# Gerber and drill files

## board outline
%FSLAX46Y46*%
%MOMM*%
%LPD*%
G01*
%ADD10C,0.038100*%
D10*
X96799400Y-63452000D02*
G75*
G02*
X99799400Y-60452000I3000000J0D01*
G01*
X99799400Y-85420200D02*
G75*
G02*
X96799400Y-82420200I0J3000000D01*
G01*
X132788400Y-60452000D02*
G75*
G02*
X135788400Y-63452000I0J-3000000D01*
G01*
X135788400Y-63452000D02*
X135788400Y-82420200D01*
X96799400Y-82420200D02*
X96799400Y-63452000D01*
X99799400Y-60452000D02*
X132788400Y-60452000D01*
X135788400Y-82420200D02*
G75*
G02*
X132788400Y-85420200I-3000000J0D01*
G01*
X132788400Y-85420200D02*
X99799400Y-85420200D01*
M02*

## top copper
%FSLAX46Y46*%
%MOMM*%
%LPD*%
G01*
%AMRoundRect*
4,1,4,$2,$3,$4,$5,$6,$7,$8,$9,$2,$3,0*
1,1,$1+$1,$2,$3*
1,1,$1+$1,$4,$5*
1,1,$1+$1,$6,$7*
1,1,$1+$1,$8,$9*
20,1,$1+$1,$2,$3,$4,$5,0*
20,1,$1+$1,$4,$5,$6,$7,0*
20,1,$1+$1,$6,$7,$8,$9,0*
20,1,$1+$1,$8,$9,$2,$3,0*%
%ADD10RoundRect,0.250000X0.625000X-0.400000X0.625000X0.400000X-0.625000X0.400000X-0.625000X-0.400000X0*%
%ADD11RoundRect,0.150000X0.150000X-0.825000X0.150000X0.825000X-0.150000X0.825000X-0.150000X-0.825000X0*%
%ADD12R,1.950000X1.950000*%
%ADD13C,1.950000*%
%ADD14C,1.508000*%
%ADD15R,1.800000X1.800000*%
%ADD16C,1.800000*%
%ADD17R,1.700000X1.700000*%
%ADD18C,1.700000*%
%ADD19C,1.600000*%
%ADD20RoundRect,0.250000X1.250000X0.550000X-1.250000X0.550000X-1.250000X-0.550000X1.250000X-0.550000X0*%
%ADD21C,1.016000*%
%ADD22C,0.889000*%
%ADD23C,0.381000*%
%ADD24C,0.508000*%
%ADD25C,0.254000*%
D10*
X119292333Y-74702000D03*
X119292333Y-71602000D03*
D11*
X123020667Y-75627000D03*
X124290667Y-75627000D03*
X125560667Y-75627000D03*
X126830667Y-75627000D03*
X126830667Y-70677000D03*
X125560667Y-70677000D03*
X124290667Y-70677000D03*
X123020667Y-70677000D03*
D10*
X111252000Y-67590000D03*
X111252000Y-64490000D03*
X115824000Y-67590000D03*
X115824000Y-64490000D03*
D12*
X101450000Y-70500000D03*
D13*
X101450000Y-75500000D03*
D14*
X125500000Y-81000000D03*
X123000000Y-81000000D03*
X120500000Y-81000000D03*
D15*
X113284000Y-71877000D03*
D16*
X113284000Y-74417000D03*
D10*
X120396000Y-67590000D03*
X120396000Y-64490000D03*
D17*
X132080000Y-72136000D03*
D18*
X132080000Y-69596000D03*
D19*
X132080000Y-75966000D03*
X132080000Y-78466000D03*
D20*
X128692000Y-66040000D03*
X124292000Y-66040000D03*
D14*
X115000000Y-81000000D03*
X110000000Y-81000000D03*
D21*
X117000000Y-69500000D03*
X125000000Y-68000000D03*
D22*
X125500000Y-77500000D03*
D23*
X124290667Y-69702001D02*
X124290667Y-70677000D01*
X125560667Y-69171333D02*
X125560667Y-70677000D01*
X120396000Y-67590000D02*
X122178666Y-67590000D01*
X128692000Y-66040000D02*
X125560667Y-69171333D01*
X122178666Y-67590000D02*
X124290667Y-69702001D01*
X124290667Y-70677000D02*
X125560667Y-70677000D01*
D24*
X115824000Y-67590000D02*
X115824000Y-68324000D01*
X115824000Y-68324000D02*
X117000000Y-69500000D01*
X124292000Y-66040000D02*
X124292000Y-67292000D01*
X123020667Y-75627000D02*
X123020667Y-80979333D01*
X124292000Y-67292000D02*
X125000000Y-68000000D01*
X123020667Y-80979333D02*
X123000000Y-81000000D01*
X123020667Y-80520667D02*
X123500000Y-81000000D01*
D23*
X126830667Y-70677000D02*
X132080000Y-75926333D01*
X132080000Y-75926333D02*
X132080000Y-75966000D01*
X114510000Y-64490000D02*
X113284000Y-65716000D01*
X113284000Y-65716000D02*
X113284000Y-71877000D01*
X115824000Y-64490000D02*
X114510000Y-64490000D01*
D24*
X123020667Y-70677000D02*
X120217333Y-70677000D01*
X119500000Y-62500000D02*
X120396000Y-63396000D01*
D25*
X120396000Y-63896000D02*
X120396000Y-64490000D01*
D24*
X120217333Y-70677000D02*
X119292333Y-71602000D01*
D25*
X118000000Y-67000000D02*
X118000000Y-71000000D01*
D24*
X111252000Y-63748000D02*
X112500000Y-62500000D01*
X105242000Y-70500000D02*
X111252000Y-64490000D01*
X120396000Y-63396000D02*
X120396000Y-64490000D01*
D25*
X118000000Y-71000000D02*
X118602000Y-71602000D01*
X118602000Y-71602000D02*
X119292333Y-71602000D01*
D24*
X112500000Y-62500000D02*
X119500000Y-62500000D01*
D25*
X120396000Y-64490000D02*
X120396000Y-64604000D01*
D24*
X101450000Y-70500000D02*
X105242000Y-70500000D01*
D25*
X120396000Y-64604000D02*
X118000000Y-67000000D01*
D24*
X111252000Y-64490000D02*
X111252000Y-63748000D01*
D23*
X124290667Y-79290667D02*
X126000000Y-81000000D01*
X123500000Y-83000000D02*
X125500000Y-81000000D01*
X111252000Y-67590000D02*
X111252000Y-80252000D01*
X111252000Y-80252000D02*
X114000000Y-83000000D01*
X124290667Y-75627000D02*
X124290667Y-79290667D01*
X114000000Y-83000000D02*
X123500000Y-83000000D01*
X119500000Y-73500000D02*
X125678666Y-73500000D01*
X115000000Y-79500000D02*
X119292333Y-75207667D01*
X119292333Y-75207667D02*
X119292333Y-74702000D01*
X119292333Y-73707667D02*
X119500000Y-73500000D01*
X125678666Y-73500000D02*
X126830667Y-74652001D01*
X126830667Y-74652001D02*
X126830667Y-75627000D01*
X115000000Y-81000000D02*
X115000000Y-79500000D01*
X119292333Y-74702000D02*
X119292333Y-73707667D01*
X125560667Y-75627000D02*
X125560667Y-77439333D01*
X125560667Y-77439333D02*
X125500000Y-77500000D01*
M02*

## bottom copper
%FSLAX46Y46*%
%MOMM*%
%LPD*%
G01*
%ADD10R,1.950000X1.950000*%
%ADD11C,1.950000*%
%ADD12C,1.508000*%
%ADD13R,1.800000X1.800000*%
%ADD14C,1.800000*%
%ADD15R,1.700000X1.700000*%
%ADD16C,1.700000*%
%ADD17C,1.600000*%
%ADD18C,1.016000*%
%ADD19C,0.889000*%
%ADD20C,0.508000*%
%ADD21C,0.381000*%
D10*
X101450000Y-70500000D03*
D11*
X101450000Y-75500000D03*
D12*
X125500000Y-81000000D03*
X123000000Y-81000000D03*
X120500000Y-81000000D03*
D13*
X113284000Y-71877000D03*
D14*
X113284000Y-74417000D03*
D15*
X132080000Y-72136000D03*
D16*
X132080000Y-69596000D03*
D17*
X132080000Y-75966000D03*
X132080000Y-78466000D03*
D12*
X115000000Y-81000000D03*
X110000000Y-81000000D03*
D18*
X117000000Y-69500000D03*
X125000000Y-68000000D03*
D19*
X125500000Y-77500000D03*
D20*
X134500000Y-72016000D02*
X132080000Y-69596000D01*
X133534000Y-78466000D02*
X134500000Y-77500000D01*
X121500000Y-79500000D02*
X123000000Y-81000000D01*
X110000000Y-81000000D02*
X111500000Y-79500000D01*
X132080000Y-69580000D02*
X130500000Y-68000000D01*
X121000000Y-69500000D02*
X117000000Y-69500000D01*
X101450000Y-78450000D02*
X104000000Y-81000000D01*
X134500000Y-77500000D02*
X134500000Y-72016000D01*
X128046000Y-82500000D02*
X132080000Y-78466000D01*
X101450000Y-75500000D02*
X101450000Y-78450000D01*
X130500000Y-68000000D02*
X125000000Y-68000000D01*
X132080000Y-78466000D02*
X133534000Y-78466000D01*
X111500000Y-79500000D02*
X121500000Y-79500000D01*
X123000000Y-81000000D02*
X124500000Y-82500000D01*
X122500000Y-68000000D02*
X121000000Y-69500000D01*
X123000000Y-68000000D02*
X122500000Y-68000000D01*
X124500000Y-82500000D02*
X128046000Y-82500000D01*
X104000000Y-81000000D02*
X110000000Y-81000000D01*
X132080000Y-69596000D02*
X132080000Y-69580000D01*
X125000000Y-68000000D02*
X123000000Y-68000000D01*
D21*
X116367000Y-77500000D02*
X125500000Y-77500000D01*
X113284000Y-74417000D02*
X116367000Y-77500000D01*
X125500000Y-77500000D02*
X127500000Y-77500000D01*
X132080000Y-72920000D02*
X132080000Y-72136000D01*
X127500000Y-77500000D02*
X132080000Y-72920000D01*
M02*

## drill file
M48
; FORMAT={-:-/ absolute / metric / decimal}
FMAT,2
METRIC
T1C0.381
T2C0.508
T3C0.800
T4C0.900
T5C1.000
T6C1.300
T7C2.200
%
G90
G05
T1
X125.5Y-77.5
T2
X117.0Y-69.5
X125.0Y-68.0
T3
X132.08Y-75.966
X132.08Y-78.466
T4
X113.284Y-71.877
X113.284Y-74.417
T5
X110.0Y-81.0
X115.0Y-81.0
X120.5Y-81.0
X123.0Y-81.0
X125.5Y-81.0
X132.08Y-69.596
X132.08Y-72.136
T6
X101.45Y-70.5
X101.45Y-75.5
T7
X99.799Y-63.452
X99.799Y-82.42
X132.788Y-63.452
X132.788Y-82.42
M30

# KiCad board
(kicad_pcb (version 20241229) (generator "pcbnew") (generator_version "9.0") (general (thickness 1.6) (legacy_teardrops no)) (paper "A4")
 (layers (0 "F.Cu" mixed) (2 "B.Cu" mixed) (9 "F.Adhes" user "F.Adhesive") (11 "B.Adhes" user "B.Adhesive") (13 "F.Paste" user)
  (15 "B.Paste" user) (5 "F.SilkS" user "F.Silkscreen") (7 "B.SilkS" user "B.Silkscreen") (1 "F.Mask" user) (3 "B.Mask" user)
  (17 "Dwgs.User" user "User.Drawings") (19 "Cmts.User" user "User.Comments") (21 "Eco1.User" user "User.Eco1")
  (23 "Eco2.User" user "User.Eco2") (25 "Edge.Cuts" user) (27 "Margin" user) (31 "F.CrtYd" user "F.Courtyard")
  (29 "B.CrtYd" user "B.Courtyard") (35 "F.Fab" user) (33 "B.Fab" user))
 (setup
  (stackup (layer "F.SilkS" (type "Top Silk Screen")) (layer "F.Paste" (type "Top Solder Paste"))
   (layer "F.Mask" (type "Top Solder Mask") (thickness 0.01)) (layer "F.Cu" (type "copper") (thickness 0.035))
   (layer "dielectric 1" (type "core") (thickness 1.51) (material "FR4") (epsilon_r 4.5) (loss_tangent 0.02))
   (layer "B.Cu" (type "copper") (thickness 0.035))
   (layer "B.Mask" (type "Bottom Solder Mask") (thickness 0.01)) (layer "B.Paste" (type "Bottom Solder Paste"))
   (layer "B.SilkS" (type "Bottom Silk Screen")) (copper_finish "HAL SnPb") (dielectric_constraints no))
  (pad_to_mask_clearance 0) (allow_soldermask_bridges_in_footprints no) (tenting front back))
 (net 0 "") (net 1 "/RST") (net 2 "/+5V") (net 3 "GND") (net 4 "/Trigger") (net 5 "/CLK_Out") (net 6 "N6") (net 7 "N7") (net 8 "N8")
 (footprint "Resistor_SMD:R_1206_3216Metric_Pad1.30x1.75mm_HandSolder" (layer "F.Cu") (at 119.292333 73.152 90)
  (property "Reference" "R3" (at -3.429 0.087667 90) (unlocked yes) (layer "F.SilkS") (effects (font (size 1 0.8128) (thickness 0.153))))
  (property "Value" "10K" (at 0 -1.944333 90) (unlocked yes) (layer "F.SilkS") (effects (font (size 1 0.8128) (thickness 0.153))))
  (pad "1" smd roundrect (at -1.55 0 90) (size 1.3 1.75) (layers "F.Cu" "F.Mask" "F.Paste") (roundrect_rratio 0.192308) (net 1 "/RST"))
  (pad "2" smd roundrect (at 1.55 0 90) (size 1.3 1.75) (layers "F.Cu" "F.Mask" "F.Paste") (roundrect_rratio 0.192308) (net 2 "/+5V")))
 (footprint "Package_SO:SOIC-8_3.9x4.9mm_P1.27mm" (layer "F.Cu") (at 124.925667 73.152 90)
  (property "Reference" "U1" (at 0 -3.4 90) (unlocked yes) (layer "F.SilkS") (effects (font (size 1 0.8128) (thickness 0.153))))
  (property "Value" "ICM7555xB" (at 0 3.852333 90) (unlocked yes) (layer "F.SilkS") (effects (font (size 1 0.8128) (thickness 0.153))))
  (pad "1" smd roundrect (at -2.475 -1.905 90) (size 1.95 0.6) (layers "F.Cu" "F.Mask" "F.Paste") (roundrect_rratio 0.25) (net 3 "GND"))
  (pad "2" smd roundrect (at -2.475 -0.635 90) (size 1.95 0.6) (layers "F.Cu" "F.Mask" "F.Paste") (roundrect_rratio 0.25) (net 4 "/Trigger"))
  (pad "3" smd roundrect (at -2.475 0.635 90) (size 1.95 0.6) (layers "F.Cu" "F.Mask" "F.Paste") (roundrect_rratio 0.25) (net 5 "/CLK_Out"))
  (pad "4" smd roundrect (at -2.475 1.905 90) (size 1.95 0.6) (layers "F.Cu" "F.Mask" "F.Paste") (roundrect_rratio 0.25) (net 1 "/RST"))
  (pad "5" smd roundrect (at 2.475 1.905 90) (size 1.95 0.6) (layers "F.Cu" "F.Mask" "F.Paste") (roundrect_rratio 0.25) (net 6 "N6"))
  (pad "6" smd roundrect (at 2.475 0.635 90) (size 1.95 0.6) (layers "F.Cu" "F.Mask" "F.Paste") (roundrect_rratio 0.25) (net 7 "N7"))
  (pad "7" smd roundrect (at 2.475 -0.635 90) (size 1.95 0.6) (layers "F.Cu" "F.Mask" "F.Paste") (roundrect_rratio 0.25) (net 7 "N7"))
  (pad "8" smd roundrect (at 2.475 -1.905 90) (size 1.95 0.6) (layers "F.Cu" "F.Mask" "F.Paste") (roundrect_rratio 0.25) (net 2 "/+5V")))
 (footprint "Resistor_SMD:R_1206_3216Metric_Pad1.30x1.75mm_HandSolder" (layer "F.Cu") (at 111.252 66.04 90)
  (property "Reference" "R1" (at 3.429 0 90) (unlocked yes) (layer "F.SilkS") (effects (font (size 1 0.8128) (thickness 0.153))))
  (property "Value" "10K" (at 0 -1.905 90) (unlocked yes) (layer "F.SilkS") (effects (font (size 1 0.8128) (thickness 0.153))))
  (pad "1" smd roundrect (at -1.55 0 90) (size 1.3 1.75) (layers "F.Cu" "F.Mask" "F.Paste") (roundrect_rratio 0.192308) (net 4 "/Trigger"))
  (pad "2" smd roundrect (at 1.55 0 90) (size 1.3 1.75) (layers "F.Cu" "F.Mask" "F.Paste") (roundrect_rratio 0.192308) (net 2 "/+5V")))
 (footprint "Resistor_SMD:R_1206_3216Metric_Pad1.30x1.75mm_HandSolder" (layer "F.Cu") (at 115.824 66.04 90)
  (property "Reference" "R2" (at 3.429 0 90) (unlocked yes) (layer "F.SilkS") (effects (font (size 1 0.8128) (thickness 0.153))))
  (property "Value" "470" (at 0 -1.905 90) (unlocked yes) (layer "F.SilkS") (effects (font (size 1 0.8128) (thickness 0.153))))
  (pad "1" smd roundrect (at -1.55 0 90) (size 1.3 1.75) (layers "F.Cu" "F.Mask" "F.Paste") (roundrect_rratio 0.192308) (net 3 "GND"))
  (pad "2" smd roundrect (at 1.55 0 90) (size 1.3 1.75) (layers "F.Cu" "F.Mask" "F.Paste") (roundrect_rratio 0.192308) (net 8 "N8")))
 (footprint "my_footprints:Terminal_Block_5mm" (layer "F.Cu") (at 101.45 73 -90)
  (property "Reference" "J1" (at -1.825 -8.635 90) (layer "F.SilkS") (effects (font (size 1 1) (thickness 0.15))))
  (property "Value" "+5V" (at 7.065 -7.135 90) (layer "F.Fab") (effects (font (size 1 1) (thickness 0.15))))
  (pad "1" thru_hole rect (at -2.5 0 270) (size 1.95 1.95) (drill 1.3) (layers "*.Cu" "*.Mask") (remove_unused_layers no) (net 2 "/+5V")
   (solder_mask_margin 0.102))
  (pad "2" thru_hole circle (at 2.5 0 270) (size 1.95 1.95) (drill 1.3) (layers "*.Cu" "*.Mask") (remove_unused_layers no) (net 3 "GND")
   (solder_mask_margin 0.102)))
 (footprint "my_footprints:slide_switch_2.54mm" (layer "F.Cu") (at 123 81 180)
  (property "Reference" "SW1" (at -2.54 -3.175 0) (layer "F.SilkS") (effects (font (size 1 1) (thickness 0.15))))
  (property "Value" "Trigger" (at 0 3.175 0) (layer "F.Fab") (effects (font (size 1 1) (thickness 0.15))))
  (pad "1" thru_hole circle (at -2.5 0 180) (size 1.508 1.508) (drill 1) (layers "*.Cu" "*.Mask") (remove_unused_layers no)
   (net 4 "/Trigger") (solder_mask_margin 0.102))
  (pad "2" thru_hole circle (at 0 0 180) (size 1.508 1.508) (drill 1) (layers "*.Cu" "*.Mask") (remove_unused_layers no) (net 3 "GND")
   (solder_mask_margin 0.102))
  (pad "3" thru_hole circle (at 2.5 0 180) (size 1.508 1.508) (drill 1) (layers "*.Cu" "*.Mask") (remove_unused_layers no)
   (solder_mask_margin 0.102)))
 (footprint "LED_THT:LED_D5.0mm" (layer "F.Cu") (at 113.284 71.877 -90)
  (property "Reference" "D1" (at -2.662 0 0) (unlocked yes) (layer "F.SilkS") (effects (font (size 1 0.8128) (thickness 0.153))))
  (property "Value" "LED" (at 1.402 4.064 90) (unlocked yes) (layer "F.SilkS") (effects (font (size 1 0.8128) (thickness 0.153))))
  (pad "1" thru_hole rect (at 0 0 270) (size 1.8 1.8) (drill 0.9) (layers "*.Cu" "*.Mask") (remove_unused_layers no) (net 8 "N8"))
  (pad "2" thru_hole circle (at 2.54 0 270) (size 1.8 1.8) (drill 0.9) (layers "*.Cu" "*.Mask") (remove_unused_layers no) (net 5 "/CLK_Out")))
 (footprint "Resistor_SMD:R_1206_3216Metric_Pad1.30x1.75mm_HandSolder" (layer "F.Cu") (at 120.396 66.04 90)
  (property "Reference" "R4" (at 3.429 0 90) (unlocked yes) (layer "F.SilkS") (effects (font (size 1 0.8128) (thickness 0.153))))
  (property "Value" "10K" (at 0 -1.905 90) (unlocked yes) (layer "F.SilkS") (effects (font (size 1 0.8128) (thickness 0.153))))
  (pad "1" smd roundrect (at -1.55 0 90) (size 1.3 1.75) (layers "F.Cu" "F.Mask" "F.Paste") (roundrect_rratio 0.192308) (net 7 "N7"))
  (pad "2" smd roundrect (at 1.55 0 90) (size 1.3 1.75) (layers "F.Cu" "F.Mask" "F.Paste") (roundrect_rratio 0.192308) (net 2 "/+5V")))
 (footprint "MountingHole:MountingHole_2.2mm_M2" (layer "F.Cu") (at 99.7994 63.452)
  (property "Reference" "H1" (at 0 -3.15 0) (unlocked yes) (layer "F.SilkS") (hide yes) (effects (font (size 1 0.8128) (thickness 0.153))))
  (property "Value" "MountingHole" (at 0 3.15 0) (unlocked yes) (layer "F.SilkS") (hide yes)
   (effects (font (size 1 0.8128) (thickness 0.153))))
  (pad "" np_thru_hole circle (at 0 0) (size 2.2 2.2) (drill 2.2) (layers "*.Cu" "*.Mask")))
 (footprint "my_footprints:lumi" (layer "F.Cu") (at 105.5 63.5)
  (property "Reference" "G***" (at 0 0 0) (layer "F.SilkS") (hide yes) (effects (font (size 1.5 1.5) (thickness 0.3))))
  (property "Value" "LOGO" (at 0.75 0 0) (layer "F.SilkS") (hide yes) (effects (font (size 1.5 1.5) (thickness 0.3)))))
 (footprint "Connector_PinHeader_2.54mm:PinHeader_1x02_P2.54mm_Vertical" (layer "F.Cu") (at 132.08 72.136 180)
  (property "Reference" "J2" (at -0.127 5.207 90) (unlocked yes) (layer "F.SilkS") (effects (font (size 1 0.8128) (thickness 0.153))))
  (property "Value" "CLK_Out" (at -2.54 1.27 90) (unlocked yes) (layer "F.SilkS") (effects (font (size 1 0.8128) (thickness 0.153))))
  (pad "1" thru_hole rect (at 0 0 180) (size 1.7 1.7) (drill 1) (layers "*.Cu" "*.Mask") (remove_unused_layers no) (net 5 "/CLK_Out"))
  (pad "2" thru_hole circle (at 0 2.54 180) (size 1.7 1.7) (drill 1) (layers "*.Cu" "*.Mask") (remove_unused_layers no) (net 3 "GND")))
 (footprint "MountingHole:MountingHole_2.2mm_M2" (layer "F.Cu") (at 132.7884 82.4202)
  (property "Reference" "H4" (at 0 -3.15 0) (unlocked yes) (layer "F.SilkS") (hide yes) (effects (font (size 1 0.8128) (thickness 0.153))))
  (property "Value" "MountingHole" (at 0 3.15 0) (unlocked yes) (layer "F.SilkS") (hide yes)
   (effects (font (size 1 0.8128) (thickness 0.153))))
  (pad "" np_thru_hole circle (at 0 0) (size 2.2 2.2) (drill 2.2) (layers "*.Cu" "*.Mask")))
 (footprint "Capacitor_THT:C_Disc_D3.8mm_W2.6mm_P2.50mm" (layer "F.Cu") (at 132.08 75.966 -90)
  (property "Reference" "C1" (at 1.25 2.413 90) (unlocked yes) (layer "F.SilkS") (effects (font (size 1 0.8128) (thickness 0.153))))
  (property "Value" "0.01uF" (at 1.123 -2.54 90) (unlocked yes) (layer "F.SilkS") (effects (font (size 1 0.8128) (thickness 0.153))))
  (pad "1" thru_hole circle (at 0 0 270) (size 1.6 1.6) (drill 0.8) (layers "*.Cu" "*.Mask") (remove_unused_layers no) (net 6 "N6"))
  (pad "2" thru_hole circle (at 2.5 0 270) (size 1.6 1.6) (drill 0.8) (layers "*.Cu" "*.Mask") (remove_unused_layers no) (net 3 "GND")))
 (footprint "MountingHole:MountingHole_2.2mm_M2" (layer "F.Cu") (at 132.7884 63.452)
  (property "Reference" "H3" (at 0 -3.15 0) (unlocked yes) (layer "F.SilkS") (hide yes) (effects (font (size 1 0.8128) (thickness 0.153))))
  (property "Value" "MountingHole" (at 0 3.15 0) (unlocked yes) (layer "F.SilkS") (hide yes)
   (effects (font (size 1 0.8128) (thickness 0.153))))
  (pad "" np_thru_hole circle (at 0 0) (size 2.2 2.2) (drill 2.2) (layers "*.Cu" "*.Mask")))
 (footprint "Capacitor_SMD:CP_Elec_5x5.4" (layer "F.Cu") (at 126.492 66.04 180)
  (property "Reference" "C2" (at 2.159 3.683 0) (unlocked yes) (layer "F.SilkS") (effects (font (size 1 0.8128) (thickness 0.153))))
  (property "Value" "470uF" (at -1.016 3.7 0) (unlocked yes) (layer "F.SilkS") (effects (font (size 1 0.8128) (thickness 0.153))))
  (pad "1" smd roundrect (at -2.2 0 180) (size 3 1.6) (layers "F.Cu" "F.Mask" "F.Paste") (roundrect_rratio 0.15625) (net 7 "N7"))
  (pad "2" smd roundrect (at 2.2 0 180) (size 3 1.6) (layers "F.Cu" "F.Mask" "F.Paste") (roundrect_rratio 0.15625) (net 3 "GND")))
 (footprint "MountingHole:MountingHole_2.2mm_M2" (layer "F.Cu") (at 99.7994 82.4202)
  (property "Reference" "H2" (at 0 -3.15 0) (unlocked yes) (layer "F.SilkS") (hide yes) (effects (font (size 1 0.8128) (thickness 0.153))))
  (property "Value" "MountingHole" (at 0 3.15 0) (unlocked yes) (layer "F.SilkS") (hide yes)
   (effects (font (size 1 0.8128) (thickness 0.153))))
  (pad "" np_thru_hole circle (at 0 0) (size 2.2 2.2) (drill 2.2) (layers "*.Cu" "*.Mask")))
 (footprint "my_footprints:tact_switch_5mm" (layer "F.Cu") (at 112.5 81 180)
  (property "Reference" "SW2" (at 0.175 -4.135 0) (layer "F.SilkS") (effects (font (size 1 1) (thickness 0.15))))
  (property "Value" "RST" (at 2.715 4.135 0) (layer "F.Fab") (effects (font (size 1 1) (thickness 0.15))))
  (pad "1" thru_hole circle (at -2.5 0 180) (size 1.508 1.508) (drill 1) (layers "*.Cu" "*.Mask") (remove_unused_layers no) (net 1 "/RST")
   (solder_mask_margin 0.102))
  (pad "2" thru_hole circle (at 2.5 0 180) (size 1.508 1.508) (drill 1) (layers "*.Cu" "*.Mask") (remove_unused_layers no) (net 3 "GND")
   (solder_mask_margin 0.102)))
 (gr_arc (start 96.7994 63.452) (mid 97.67808 61.33068) (end 99.7994 60.452) (stroke (width 0.0381) (type default)) (layer "Edge.Cuts"))
 (gr_arc (start 99.7994 85.4202) (mid 97.67808 84.54152) (end 96.7994 82.4202) (stroke (width 0.0381) (type default)) (layer "Edge.Cuts"))
 (gr_arc (start 132.7884 60.452) (mid 134.90972 61.33068) (end 135.7884 63.452) (stroke (width 0.0381) (type default)) (layer "Edge.Cuts"))
 (gr_line (start 135.7884 63.452) (end 135.7884 82.4202) (stroke (width 0.0381) (type default)) (layer "Edge.Cuts"))
 (gr_line (start 96.7994 82.4202) (end 96.7994 63.452) (stroke (width 0.0381) (type default)) (layer "Edge.Cuts"))
 (gr_line (start 99.7994 60.452) (end 132.7884 60.452) (stroke (width 0.0381) (type default)) (layer "Edge.Cuts"))
 (gr_arc (start 135.7884 82.4202) (mid 134.90972 84.54152) (end 132.7884 85.4202) (stroke (width 0.0381) (type default)) (layer "Edge.Cuts"))
 (gr_line (start 132.7884 85.4202) (end 99.7994 85.4202) (stroke (width 0.0381) (type default)) (layer "Edge.Cuts"))
 (segment (start 124.290667 69.702001) (end 124.290667 70.677) (width 0.381) (layer "F.Cu") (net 7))
 (segment (start 125.560667 69.171333) (end 125.560667 70.677) (width 0.381) (layer "F.Cu") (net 7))
 (segment (start 120.396 67.59) (end 122.178666 67.59) (width 0.381) (layer "F.Cu") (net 7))
 (segment (start 128.692 66.04) (end 125.560667 69.171333) (width 0.381) (layer "F.Cu") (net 7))
 (segment (start 122.178666 67.59) (end 124.290667 69.702001) (width 0.381) (layer "F.Cu") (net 7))
 (segment (start 124.290667 70.677) (end 125.560667 70.677) (width 0.381) (layer "F.Cu") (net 7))
 (segment (start 115.824 67.59) (end 115.824 68.324) (width 0.508) (layer "F.Cu") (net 3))
 (segment (start 115.824 68.324) (end 117 69.5) (width 0.508) (layer "F.Cu") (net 3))
 (segment (start 124.292 66.04) (end 124.292 67.292) (width 0.508) (layer "F.Cu") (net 3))
 (segment (start 123.020667 75.627) (end 123.020667 80.979333) (width 0.508) (layer "F.Cu") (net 3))
 (segment (start 124.292 67.292) (end 125 68) (width 0.508) (layer "F.Cu") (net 3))
 (segment (start 123.020667 80.979333) (end 123 81) (width 0.508) (layer "F.Cu") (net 3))
 (segment (start 123.020667 80.520667) (end 123.5 81) (width 0.508) (layer "F.Cu") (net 3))
 (via (at 117 69.5) (size 1.016) (drill 0.508) (layers "F.Cu" "B.Cu") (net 3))
 (via (at 125 68) (size 1.016) (drill 0.508) (layers "F.Cu" "B.Cu") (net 3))
 (segment (start 134.5 72.016) (end 132.08 69.596) (width 0.508) (layer "B.Cu") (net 3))
 (segment (start 133.534 78.466) (end 134.5 77.5) (width 0.508) (layer "B.Cu") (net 3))
 (segment (start 121.5 79.5) (end 123 81) (width 0.508) (layer "B.Cu") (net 3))
 (segment (start 110 81) (end 111.5 79.5) (width 0.508) (layer "B.Cu") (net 3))
 (segment (start 132.08 69.58) (end 130.5 68) (width 0.508) (layer "B.Cu") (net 3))
 (segment (start 121 69.5) (end 117 69.5) (width 0.508) (layer "B.Cu") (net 3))
 (segment (start 101.45 78.45) (end 104 81) (width 0.508) (layer "B.Cu") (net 3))
 (segment (start 134.5 77.5) (end 134.5 72.016) (width 0.508) (layer "B.Cu") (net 3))
 (segment (start 128.046 82.5) (end 132.08 78.466) (width 0.508) (layer "B.Cu") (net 3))
 (segment (start 101.45 75.5) (end 101.45 78.45) (width 0.508) (layer "B.Cu") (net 3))
 (segment (start 130.5 68) (end 125 68) (width 0.508) (layer "B.Cu") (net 3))
 (segment (start 132.08 78.466) (end 133.534 78.466) (width 0.508) (layer "B.Cu") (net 3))
 (segment (start 111.5 79.5) (end 121.5 79.5) (width 0.508) (layer "B.Cu") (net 3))
 (segment (start 123 81) (end 124.5 82.5) (width 0.508) (layer "B.Cu") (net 3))
 (segment (start 122.5 68) (end 121 69.5) (width 0.508) (layer "B.Cu") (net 3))
 (segment (start 123 68) (end 122.5 68) (width 0.508) (layer "B.Cu") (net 3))
 (segment (start 124.5 82.5) (end 128.046 82.5) (width 0.508) (layer "B.Cu") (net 3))
 (segment (start 104 81) (end 110 81) (width 0.508) (layer "B.Cu") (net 3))
 (segment (start 132.08 69.596) (end 132.08 69.58) (width 0.508) (layer "B.Cu") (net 3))
 (segment (start 125 68) (end 123 68) (width 0.508) (layer "B.Cu") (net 3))
 (segment (start 126.830667 70.677) (end 132.08 75.926333) (width 0.381) (layer "F.Cu") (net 6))
 (segment (start 132.08 75.926333) (end 132.08 75.966) (width 0.381) (layer "F.Cu") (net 6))
 (segment (start 114.51 64.49) (end 113.284 65.716) (width 0.381) (layer "F.Cu") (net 8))
 (segment (start 113.284 65.716) (end 113.284 71.877) (width 0.381) (layer "F.Cu") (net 8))
 (segment (start 115.824 64.49) (end 114.51 64.49) (width 0.381) (layer "F.Cu") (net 8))
 (segment (start 123.020667 70.677) (end 120.217333 70.677) (width 0.508) (layer "F.Cu") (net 2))
 (segment (start 119.5 62.5) (end 120.396 63.396) (width 0.508) (layer "F.Cu") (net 2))
 (segment (start 120.396 63.896) (end 120.396 64.49) (width 0.254) (layer "F.Cu") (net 2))
 (segment (start 120.217333 70.677) (end 119.292333 71.602) (width 0.508) (layer "F.Cu") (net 2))
 (segment (start 118 67) (end 118 71) (width 0.254) (layer "F.Cu") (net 2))
 (segment (start 111.252 63.748) (end 112.5 62.5) (width 0.508) (layer "F.Cu") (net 2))
 (segment (start 105.242 70.5) (end 111.252 64.49) (width 0.508) (layer "F.Cu") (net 2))
 (segment (start 120.396 63.396) (end 120.396 64.49) (width 0.508) (layer "F.Cu") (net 2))
 (segment (start 118 71) (end 118.602 71.602) (width 0.254) (layer "F.Cu") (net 2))
 (segment (start 118.602 71.602) (end 119.292333 71.602) (width 0.254) (layer "F.Cu") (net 2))
 (segment (start 112.5 62.5) (end 119.5 62.5) (width 0.508) (layer "F.Cu") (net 2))
 (segment (start 120.396 64.49) (end 120.396 64.604) (width 0.254) (layer "F.Cu") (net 2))
 (segment (start 101.45 70.5) (end 105.242 70.5) (width 0.508) (layer "F.Cu") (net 2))
 (segment (start 120.396 64.604) (end 118 67) (width 0.254) (layer "F.Cu") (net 2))
 (segment (start 111.252 64.49) (end 111.252 63.748) (width 0.508) (layer "F.Cu") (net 2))
 (segment (start 124.290667 79.290667) (end 126 81) (width 0.381) (layer "F.Cu") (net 4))
 (segment (start 123.5 83) (end 125.5 81) (width 0.381) (layer "F.Cu") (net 4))
 (segment (start 111.252 67.59) (end 111.252 80.252) (width 0.381) (layer "F.Cu") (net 4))
 (segment (start 111.252 80.252) (end 114 83) (width 0.381) (layer "F.Cu") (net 4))
 (segment (start 124.290667 75.627) (end 124.290667 79.290667) (width 0.381) (layer "F.Cu") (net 4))
 (segment (start 114 83) (end 123.5 83) (width 0.381) (layer "F.Cu") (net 4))
 (segment (start 119.5 73.5) (end 125.678666 73.5) (width 0.381) (layer "F.Cu") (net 1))
 (segment (start 115 79.5) (end 119.292333 75.207667) (width 0.381) (layer "F.Cu") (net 1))
 (segment (start 119.292333 75.207667) (end 119.292333 74.702) (width 0.381) (layer "F.Cu") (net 1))
 (segment (start 119.292333 73.707667) (end 119.5 73.5) (width 0.381) (layer "F.Cu") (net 1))
 (segment (start 125.678666 73.5) (end 126.830667 74.652001) (width 0.381) (layer "F.Cu") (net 1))
 (segment (start 126.830667 74.652001) (end 126.830667 75.627) (width 0.381) (layer "F.Cu") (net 1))
 (segment (start 115 81) (end 115 79.5) (width 0.381) (layer "F.Cu") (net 1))
 (segment (start 119.292333 74.702) (end 119.292333 73.707667) (width 0.381) (layer "F.Cu") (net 1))
 (segment (start 125.560667 75.627) (end 125.560667 77.439333) (width 0.381) (layer "F.Cu") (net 5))
 (segment (start 125.560667 77.439333) (end 125.5 77.5) (width 0.381) (layer "F.Cu") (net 5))
 (via (at 125.5 77.5) (size 0.889) (drill 0.381) (layers "F.Cu" "B.Cu") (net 5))
 (segment (start 116.367 77.5) (end 125.5 77.5) (width 0.381) (layer "B.Cu") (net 5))
 (segment (start 113.284 74.417) (end 116.367 77.5) (width 0.381) (layer "B.Cu") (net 5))
 (segment (start 125.5 77.5) (end 127.5 77.5) (width 0.381) (layer "B.Cu") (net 5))
 (segment (start 132.08 72.92) (end 132.08 72.136) (width 0.381) (layer "B.Cu") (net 5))
 (segment (start 127.5 77.5) (end 132.08 72.92) (width 0.381) (layer "B.Cu") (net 5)))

